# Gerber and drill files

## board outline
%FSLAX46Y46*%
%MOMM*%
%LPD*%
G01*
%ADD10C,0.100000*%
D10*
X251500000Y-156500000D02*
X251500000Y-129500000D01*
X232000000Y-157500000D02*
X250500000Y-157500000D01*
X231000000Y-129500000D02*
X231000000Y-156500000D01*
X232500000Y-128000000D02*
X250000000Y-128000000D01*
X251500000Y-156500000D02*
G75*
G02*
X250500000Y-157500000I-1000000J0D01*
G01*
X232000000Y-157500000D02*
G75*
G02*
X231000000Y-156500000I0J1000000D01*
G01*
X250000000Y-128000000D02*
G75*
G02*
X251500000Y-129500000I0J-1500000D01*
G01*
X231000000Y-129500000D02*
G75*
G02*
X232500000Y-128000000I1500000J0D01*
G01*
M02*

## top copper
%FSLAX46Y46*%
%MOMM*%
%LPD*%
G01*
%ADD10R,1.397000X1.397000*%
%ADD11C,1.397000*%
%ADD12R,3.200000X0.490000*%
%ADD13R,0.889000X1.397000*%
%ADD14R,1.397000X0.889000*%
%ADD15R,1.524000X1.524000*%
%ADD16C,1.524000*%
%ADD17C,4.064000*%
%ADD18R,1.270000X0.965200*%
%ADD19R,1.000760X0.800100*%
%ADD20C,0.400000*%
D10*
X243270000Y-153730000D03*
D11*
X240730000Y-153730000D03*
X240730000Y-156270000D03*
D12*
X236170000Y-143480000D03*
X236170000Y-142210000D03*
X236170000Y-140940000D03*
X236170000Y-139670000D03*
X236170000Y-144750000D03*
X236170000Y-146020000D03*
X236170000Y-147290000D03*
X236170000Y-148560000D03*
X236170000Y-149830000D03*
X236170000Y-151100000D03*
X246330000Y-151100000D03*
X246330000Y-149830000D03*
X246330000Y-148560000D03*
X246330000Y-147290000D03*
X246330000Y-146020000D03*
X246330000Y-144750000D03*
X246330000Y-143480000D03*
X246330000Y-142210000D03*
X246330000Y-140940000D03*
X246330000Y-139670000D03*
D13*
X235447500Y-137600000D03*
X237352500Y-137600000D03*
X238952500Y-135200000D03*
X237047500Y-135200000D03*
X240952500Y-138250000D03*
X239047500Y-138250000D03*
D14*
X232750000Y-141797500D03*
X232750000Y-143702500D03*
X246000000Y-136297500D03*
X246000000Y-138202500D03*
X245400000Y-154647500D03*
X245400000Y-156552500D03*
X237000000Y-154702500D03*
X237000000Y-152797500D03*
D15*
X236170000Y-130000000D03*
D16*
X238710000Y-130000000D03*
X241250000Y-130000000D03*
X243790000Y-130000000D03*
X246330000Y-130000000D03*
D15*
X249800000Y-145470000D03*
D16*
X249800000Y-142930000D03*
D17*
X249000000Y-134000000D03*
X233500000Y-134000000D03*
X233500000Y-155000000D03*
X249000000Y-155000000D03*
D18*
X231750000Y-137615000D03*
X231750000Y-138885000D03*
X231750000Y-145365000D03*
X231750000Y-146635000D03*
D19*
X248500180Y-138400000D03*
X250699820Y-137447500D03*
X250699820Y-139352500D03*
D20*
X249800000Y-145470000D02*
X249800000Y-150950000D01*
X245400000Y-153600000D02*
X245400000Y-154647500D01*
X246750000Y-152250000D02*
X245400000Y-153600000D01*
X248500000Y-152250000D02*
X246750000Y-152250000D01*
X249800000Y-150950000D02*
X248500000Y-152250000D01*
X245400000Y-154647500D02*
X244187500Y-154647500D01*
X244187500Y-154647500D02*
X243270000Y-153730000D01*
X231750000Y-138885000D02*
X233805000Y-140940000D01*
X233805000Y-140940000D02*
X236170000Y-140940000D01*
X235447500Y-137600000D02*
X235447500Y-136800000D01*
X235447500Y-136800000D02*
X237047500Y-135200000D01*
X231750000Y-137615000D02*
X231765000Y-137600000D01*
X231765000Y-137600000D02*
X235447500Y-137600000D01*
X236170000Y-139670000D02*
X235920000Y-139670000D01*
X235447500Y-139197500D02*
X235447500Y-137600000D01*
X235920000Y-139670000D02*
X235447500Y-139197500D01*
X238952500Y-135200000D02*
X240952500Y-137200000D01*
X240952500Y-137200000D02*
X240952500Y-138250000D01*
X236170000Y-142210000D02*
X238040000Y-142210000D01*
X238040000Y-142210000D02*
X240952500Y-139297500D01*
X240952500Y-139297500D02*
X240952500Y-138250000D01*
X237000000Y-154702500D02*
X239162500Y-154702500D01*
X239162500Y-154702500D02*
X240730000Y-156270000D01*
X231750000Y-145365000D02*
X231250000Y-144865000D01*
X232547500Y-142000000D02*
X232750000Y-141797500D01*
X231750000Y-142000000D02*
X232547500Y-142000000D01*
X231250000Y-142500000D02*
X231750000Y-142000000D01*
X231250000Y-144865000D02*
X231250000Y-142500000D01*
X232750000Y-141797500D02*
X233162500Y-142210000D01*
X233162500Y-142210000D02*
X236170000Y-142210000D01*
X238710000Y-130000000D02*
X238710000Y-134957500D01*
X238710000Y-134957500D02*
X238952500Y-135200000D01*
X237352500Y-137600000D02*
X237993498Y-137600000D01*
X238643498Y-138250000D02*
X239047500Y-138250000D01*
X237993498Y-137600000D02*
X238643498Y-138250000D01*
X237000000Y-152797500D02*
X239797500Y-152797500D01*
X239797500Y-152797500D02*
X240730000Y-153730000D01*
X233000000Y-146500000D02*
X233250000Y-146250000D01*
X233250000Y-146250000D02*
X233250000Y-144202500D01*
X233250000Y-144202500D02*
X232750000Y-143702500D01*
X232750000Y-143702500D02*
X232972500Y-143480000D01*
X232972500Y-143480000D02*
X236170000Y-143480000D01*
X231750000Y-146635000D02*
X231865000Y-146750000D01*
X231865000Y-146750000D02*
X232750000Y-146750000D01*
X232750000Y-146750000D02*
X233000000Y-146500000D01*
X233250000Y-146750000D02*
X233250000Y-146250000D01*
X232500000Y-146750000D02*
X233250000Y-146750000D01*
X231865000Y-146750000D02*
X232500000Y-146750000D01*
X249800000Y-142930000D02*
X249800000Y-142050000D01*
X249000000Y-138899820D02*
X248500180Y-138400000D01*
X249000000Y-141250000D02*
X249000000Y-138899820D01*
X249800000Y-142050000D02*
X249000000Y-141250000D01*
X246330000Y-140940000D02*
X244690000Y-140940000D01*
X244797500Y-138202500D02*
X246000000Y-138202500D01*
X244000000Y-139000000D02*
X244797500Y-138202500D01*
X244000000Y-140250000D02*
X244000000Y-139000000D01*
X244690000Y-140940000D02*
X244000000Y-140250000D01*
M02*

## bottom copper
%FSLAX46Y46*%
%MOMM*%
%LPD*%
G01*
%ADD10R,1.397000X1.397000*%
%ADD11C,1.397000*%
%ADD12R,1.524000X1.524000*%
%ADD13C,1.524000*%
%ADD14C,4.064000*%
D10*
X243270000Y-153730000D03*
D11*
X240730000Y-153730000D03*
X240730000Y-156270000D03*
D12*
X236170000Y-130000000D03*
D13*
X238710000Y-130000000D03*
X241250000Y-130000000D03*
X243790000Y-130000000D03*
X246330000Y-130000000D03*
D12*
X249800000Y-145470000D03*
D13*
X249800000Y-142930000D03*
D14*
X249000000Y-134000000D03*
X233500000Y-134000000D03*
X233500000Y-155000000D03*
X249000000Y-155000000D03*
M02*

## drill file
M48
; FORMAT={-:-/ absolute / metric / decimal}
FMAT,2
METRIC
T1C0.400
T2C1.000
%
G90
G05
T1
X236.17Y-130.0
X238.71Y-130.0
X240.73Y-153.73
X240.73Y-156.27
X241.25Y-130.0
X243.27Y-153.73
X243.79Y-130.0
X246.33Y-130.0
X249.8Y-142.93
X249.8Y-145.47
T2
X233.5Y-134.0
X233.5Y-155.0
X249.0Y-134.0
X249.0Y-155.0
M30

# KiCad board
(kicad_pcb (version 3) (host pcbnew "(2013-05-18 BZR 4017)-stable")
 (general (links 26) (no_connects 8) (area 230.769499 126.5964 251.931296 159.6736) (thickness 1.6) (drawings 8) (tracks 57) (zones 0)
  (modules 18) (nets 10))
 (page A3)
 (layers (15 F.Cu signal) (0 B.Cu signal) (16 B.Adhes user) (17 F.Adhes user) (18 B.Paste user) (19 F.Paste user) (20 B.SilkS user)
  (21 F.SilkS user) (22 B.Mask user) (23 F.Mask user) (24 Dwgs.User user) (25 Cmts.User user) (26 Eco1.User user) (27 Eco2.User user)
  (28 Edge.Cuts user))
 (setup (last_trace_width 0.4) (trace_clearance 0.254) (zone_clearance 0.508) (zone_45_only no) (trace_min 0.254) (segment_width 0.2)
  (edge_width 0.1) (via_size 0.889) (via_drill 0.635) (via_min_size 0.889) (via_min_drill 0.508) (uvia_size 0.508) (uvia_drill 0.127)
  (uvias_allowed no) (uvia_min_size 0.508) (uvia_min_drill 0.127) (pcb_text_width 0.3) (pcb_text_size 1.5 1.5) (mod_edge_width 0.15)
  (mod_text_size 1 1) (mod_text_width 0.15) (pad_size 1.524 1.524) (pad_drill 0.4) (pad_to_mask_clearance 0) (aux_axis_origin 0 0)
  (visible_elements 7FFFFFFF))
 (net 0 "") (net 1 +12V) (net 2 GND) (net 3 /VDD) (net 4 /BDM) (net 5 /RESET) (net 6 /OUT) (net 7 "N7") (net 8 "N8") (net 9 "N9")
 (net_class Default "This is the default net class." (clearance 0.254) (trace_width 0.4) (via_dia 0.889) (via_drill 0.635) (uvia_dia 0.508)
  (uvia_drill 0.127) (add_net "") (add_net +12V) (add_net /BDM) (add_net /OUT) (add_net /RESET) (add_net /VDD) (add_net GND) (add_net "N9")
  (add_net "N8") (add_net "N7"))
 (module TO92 (layer F.Cu) (at 242 155)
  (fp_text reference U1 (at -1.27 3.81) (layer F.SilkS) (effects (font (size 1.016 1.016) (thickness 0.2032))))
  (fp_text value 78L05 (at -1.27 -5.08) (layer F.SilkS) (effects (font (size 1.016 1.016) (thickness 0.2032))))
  (pad 1 thru_hole rect (at 1.27 -1.27) (size 1.397 1.397) (drill 0.4) (layers *.Cu *.Mask F.SilkS) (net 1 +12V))
  (pad 2 thru_hole circle (at -1.27 -1.27) (size 1.397 1.397) (drill 0.4) (layers *.Cu *.Mask F.SilkS) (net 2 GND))
  (pad 3 thru_hole circle (at -1.27 1.27) (size 1.397 1.397) (drill 0.4) (layers *.Cu *.Mask F.SilkS) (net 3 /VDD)))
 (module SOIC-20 (layer F.Cu) (at 241.25 144.75)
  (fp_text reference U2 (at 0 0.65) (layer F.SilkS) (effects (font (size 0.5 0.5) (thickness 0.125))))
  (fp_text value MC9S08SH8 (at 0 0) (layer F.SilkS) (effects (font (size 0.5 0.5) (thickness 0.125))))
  (pad 4 smd rect (at -5.08 -1.27) (size 3.2 0.49) (layers F.Cu F.Paste F.Mask) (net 2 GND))
  (pad 3 smd rect (at -5.08 -2.54) (size 3.2 0.49) (layers F.Cu F.Paste F.Mask) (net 3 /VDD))
  (pad 2 smd rect (at -5.08 -3.81) (size 3.2 0.49) (layers F.Cu F.Paste F.Mask) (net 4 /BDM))
  (pad 1 smd rect (at -5.08 -5.08) (size 3.2 0.49) (layers F.Cu F.Paste F.Mask) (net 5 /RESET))
  (pad 5 smd rect (at -5.08 0) (size 3.2 0.49) (layers F.Cu F.Paste F.Mask))
  (pad 6 smd rect (at -5.08 1.27) (size 3.2 0.49) (layers F.Cu F.Paste F.Mask))
  (pad 7 smd rect (at -5.08 2.54) (size 3.2 0.49) (layers F.Cu F.Paste F.Mask))
  (pad 8 smd rect (at -5.08 3.81) (size 3.2 0.49) (layers F.Cu F.Paste F.Mask))
  (pad 9 smd rect (at -5.08 5.08) (size 3.2 0.49) (layers F.Cu F.Paste F.Mask))
  (pad 10 smd rect (at -5.08 6.35) (size 3.2 0.49) (layers F.Cu F.Paste F.Mask))
  (pad 11 smd rect (at 5.08 6.35) (size 3.2 0.49) (layers F.Cu F.Paste F.Mask))
  (pad 12 smd rect (at 5.08 5.08) (size 3.2 0.49) (layers F.Cu F.Paste F.Mask) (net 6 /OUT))
  (pad 13 smd rect (at 5.08 3.81) (size 3.2 0.49) (layers F.Cu F.Paste F.Mask))
  (pad 14 smd rect (at 5.08 2.54) (size 3.2 0.49) (layers F.Cu F.Paste F.Mask))
  (pad 15 smd rect (at 5.08 1.27) (size 3.2 0.49) (layers F.Cu F.Paste F.Mask))
  (pad 16 smd rect (at 5.08 0) (size 3.2 0.49) (layers F.Cu F.Paste F.Mask))
  (pad 17 smd rect (at 5.08 -1.27) (size 3.2 0.49) (layers F.Cu F.Paste F.Mask))
  (pad 18 smd rect (at 5.08 -2.54) (size 3.2 0.49) (layers F.Cu F.Paste F.Mask))
  (pad 19 smd rect (at 5.08 -3.81) (size 3.2 0.49) (layers F.Cu F.Paste F.Mask) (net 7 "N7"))
  (pad 20 smd rect (at 5.08 -5.08) (size 3.2 0.49) (layers F.Cu F.Paste F.Mask)))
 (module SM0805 (layer F.Cu) (at 236.4 137.6)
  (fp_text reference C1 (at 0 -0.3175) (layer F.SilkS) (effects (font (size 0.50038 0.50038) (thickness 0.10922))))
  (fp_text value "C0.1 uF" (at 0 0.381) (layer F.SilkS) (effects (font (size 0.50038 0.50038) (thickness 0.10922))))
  (pad 1 smd rect (at -0.9525 0) (size 0.889 1.397) (layers F.Cu F.Paste F.Mask) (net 5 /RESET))
  (pad 2 smd rect (at 0.9525 0) (size 0.889 1.397) (layers F.Cu F.Paste F.Mask) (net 2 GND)))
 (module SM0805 (layer F.Cu) (at 238 135.2 180)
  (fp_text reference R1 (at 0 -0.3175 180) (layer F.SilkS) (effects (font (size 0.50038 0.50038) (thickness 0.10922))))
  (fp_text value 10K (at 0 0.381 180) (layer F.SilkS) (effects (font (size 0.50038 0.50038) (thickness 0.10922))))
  (pad 1 smd rect (at -0.9525 0 180) (size 0.889 1.397) (layers F.Cu F.Paste F.Mask) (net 3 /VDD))
  (pad 2 smd rect (at 0.9525 0 180) (size 0.889 1.397) (layers F.Cu F.Paste F.Mask) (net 5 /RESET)))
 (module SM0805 (layer F.Cu) (at 240 138.25 180)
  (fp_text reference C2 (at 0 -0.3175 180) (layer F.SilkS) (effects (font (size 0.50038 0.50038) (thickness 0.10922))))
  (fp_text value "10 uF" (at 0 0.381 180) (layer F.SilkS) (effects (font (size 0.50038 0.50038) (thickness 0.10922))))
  (pad 1 smd rect (at -0.9525 0 180) (size 0.889 1.397) (layers F.Cu F.Paste F.Mask) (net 3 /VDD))
  (pad 2 smd rect (at 0.9525 0 180) (size 0.889 1.397) (layers F.Cu F.Paste F.Mask) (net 2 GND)))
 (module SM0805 (layer F.Cu) (at 232.75 142.75 270)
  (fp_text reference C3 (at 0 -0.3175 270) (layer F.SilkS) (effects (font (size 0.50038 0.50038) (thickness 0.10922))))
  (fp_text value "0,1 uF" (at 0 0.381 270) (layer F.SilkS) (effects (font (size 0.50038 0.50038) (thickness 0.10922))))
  (pad 1 smd rect (at -0.9525 0 270) (size 0.889 1.397) (layers F.Cu F.Paste F.Mask) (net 3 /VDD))
  (pad 2 smd rect (at 0.9525 0 270) (size 0.889 1.397) (layers F.Cu F.Paste F.Mask) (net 2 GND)))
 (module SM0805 (layer F.Cu) (at 246 137.25 270)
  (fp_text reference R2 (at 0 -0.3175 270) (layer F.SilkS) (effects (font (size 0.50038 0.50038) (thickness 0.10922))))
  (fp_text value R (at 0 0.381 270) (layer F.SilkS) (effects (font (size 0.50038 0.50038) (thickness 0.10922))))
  (pad 1 smd rect (at -0.9525 0 270) (size 0.889 1.397) (layers F.Cu F.Paste F.Mask) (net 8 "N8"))
  (pad 2 smd rect (at 0.9525 0 270) (size 0.889 1.397) (layers F.Cu F.Paste F.Mask) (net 7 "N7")))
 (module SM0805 (layer F.Cu) (at 245.4 155.6 270)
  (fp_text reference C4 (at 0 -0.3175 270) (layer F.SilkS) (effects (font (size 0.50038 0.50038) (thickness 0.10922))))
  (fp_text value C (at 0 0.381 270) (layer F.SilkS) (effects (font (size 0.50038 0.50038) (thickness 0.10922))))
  (pad 1 smd rect (at -0.9525 0 270) (size 0.889 1.397) (layers F.Cu F.Paste F.Mask) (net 1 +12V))
  (pad 2 smd rect (at 0.9525 0 270) (size 0.889 1.397) (layers F.Cu F.Paste F.Mask) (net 2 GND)))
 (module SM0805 (layer F.Cu) (at 237 153.75 90)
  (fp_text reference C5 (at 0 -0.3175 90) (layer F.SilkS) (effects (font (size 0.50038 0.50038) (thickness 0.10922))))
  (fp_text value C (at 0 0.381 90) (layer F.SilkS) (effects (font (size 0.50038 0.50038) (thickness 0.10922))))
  (pad 1 smd rect (at -0.9525 0 90) (size 0.889 1.397) (layers F.Cu F.Paste F.Mask) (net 3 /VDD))
  (pad 2 smd rect (at 0.9525 0 90) (size 0.889 1.397) (layers F.Cu F.Paste F.Mask) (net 2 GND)))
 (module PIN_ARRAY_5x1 (layer F.Cu) (at 241.25 130)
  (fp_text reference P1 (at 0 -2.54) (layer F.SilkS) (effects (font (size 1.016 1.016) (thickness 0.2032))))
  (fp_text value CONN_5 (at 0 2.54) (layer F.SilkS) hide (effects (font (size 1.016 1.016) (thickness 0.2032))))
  (pad 1 thru_hole rect (at -5.08 0) (size 1.524 1.524) (drill 0.4) (layers *.Cu *.Mask F.SilkS))
  (pad 2 thru_hole circle (at -2.54 0) (size 1.524 1.524) (drill 0.4) (layers *.Cu *.Mask F.SilkS) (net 3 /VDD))
  (pad 3 thru_hole circle (at 0 0) (size 1.524 1.524) (drill 0.4) (layers *.Cu *.Mask F.SilkS))
  (pad 4 thru_hole circle (at 2.54 0) (size 1.524 1.524) (drill 0.4) (layers *.Cu *.Mask F.SilkS) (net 6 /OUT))
  (pad 5 thru_hole circle (at 5.08 0) (size 1.524 1.524) (drill 0.4) (layers *.Cu *.Mask F.SilkS) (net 2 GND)))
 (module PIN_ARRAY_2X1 (layer F.Cu) (at 249.8 144.2 90)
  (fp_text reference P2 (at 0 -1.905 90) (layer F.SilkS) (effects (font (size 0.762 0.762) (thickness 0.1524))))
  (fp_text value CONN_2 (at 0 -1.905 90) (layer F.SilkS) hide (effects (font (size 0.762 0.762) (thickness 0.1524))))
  (pad 1 thru_hole rect (at -1.27 0 90) (size 1.524 1.524) (drill 0.4) (layers *.Cu *.Mask F.SilkS) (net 1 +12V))
  (pad 2 thru_hole circle (at 1.27 0 90) (size 1.524 1.524) (drill 0.4) (layers *.Cu *.Mask F.SilkS) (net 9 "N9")))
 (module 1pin (layer F.Cu) (at 249 134)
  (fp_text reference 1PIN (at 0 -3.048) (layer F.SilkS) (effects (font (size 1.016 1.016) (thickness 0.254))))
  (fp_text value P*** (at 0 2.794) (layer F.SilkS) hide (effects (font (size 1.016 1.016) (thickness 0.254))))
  (pad 1 thru_hole circle (at 0 0) (size 4.064 4.064) (drill 1) (layers *.Cu *.Mask F.SilkS)))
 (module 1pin (layer F.Cu) (at 233.5 134)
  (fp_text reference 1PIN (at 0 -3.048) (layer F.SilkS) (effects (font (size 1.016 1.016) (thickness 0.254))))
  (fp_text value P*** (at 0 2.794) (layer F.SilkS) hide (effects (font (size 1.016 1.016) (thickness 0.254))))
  (pad 1 thru_hole circle (at 0 0) (size 4.064 4.064) (drill 1) (layers *.Cu *.Mask F.SilkS)))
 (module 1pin (layer F.Cu) (at 233.5 155)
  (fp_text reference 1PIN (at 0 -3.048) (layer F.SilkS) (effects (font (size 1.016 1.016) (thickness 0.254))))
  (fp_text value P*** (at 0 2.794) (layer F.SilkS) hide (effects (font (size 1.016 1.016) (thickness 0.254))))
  (pad 1 thru_hole circle (at 0 0) (size 4.064 4.064) (drill 1) (layers *.Cu *.Mask F.SilkS)))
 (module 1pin (layer F.Cu) (at 249 155)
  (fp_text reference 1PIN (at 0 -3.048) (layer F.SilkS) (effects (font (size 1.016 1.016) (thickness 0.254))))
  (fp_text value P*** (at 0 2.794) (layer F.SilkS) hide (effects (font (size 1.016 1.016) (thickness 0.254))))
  (pad 1 thru_hole circle (at 0 0) (size 4.064 4.064) (drill 1) (layers *.Cu *.Mask F.SilkS)))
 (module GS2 (layer F.Cu) (at 231.75 138.25)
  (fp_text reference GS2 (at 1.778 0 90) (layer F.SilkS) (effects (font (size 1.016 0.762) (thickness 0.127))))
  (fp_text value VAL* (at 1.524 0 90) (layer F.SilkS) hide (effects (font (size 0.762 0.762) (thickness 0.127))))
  (pad 1 smd rect (at 0 -0.635) (size 1.27 0.9652) (layers F.Cu F.Paste F.Mask) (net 5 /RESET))
  (pad 2 smd rect (at 0 0.635) (size 1.27 0.9652) (layers F.Cu F.Paste F.Mask) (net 4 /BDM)))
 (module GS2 (layer F.Cu) (at 231.75 146)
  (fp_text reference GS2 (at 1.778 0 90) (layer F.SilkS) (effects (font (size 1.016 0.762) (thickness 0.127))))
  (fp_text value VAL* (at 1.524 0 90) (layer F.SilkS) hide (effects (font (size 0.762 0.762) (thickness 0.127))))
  (pad 1 smd rect (at 0 -0.635) (size 1.27 0.9652) (layers F.Cu F.Paste F.Mask) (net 3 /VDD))
  (pad 2 smd rect (at 0 0.635) (size 1.27 0.9652) (layers F.Cu F.Paste F.Mask) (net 2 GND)))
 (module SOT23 (layer F.Cu) (at 249.6 138.4 90)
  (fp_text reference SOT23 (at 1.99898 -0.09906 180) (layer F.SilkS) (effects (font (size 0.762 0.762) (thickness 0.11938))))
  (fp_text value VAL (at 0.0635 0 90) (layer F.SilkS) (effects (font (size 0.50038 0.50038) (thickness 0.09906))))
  (pad 3 smd rect (at 0 -1.09982 90) (size 0.8001 1.00076) (layers F.Cu F.Paste F.Mask) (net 9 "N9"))
  (pad 2 smd rect (at 0.9525 1.09982 90) (size 0.8001 1.00076) (layers F.Cu F.Paste F.Mask) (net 2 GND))
  (pad 1 smd rect (at -0.9525 1.09982 90) (size 0.8001 1.00076) (layers F.Cu F.Paste F.Mask) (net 8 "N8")))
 (gr_line (start 251.5 156.5) (end 251.5 129.5) (angle 90) (layer Edge.Cuts) (width 0.1))
 (gr_line (start 232 157.5) (end 250.5 157.5) (angle 90) (layer Edge.Cuts) (width 0.1))
 (gr_line (start 231 129.5) (end 231 156.5) (angle 90) (layer Edge.Cuts) (width 0.1))
 (gr_line (start 232.5 128) (end 250 128) (angle 90) (layer Edge.Cuts) (width 0.1))
 (gr_arc (start 250.5 156.5) (end 251.5 156.5) (angle 90) (layer Edge.Cuts) (width 0.1))
 (gr_arc (start 232 156.5) (end 232 157.5) (angle 90) (layer Edge.Cuts) (width 0.1))
 (gr_arc (start 250 129.5) (end 250 128) (angle 90) (layer Edge.Cuts) (width 0.1))
 (gr_arc (start 232.5 129.5) (end 231 129.5) (angle 90) (layer Edge.Cuts) (width 0.1))
 (segment (start 249.8 145.47) (end 249.8 150.95) (width 0.4) (layer F.Cu) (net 1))
 (segment (start 245.4 153.6) (end 245.4 154.6475) (width 0.4) (layer F.Cu) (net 1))
 (segment (start 246.75 152.25) (end 245.4 153.6) (width 0.4) (layer F.Cu) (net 1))
 (segment (start 248.5 152.25) (end 246.75 152.25) (width 0.4) (layer F.Cu) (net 1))
 (segment (start 249.8 150.95) (end 248.5 152.25) (width 0.4) (layer F.Cu) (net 1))
 (segment (start 245.4 154.6475) (end 244.1875 154.6475) (width 0.4) (layer F.Cu) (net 1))
 (segment (start 244.1875 154.6475) (end 243.27 153.73) (width 0.4) (layer F.Cu) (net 1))
 (segment (start 231.75 138.885) (end 233.805 140.94) (width 0.4) (layer F.Cu) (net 4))
 (segment (start 233.805 140.94) (end 236.17 140.94) (width 0.4) (layer F.Cu) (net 4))
 (segment (start 235.4475 137.6) (end 235.4475 136.8) (width 0.4) (layer F.Cu) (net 5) (status 400000))
 (segment (start 235.4475 136.8) (end 237.0475 135.2) (width 0.4) (layer F.Cu) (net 5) (status 800000))
 (segment (start 231.75 137.615) (end 231.765 137.6) (width 0.4) (layer F.Cu) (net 5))
 (segment (start 231.765 137.6) (end 235.4475 137.6) (width 0.4) (layer F.Cu) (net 5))
 (segment (start 236.17 139.67) (end 235.92 139.67) (width 0.4) (layer F.Cu) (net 5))
 (segment (start 235.4475 139.1975) (end 235.4475 137.6) (width 0.4) (layer F.Cu) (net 5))
 (segment (start 235.92 139.67) (end 235.4475 139.1975) (width 0.4) (layer F.Cu) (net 5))
 (segment (start 238.9525 135.2) (end 240.9525 137.2) (width 0.4) (layer F.Cu) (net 3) (status 400000))
 (segment (start 240.9525 137.2) (end 240.9525 138.25) (width 0.4) (layer F.Cu) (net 3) (status 800000))
 (segment (start 236.17 142.21) (end 238.04 142.21) (width 0.4) (layer F.Cu) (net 3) (status 400000))
 (segment (start 238.04 142.21) (end 240.9525 139.2975) (width 0.4) (layer F.Cu) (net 3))
 (segment (start 240.9525 139.2975) (end 240.9525 138.25) (width 0.4) (layer F.Cu) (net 3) (status 800000))
 (segment (start 237 154.7025) (end 239.1625 154.7025) (width 0.4) (layer F.Cu) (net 3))
 (segment (start 239.1625 154.7025) (end 240.73 156.27) (width 0.4) (layer F.Cu) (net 3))
 (segment (start 231.75 145.365) (end 231.25 144.865) (width 0.4) (layer F.Cu) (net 3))
 (segment (start 232.5475 142) (end 232.75 141.7975) (width 0.4) (layer F.Cu) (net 3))
 (segment (start 231.75 142) (end 232.5475 142) (width 0.4) (layer F.Cu) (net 3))
 (segment (start 231.25 142.5) (end 231.75 142) (width 0.4) (layer F.Cu) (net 3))
 (segment (start 231.25 144.865) (end 231.25 142.5) (width 0.4) (layer F.Cu) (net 3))
 (segment (start 232.75 141.7975) (end 233.1625 142.21) (width 0.4) (layer F.Cu) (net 3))
 (segment (start 233.1625 142.21) (end 236.17 142.21) (width 0.4) (layer F.Cu) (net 3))
 (segment (start 238.71 130) (end 238.71 134.9575) (width 0.4) (layer F.Cu) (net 3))
 (segment (start 238.71 134.9575) (end 238.9525 135.2) (width 0.4) (layer F.Cu) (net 3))
 (segment (start 237.3525 137.6) (end 237.993498 137.6) (width 0.4) (layer F.Cu) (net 2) (status 400000))
 (segment (start 238.643498 138.25) (end 239.0475 138.25) (width 0.4) (layer F.Cu) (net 2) (status C00000))
 (segment (start 237.993498 137.6) (end 238.643498 138.25) (width 0.4) (layer F.Cu) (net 2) (status 800000))
 (segment (start 237 152.7975) (end 239.7975 152.7975) (width 0.4) (layer F.Cu) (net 2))
 (segment (start 239.7975 152.7975) (end 240.73 153.73) (width 0.4) (layer F.Cu) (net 2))
 (segment (start 233 146.5) (end 233.25 146.25) (width 0.4) (layer F.Cu) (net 2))
 (segment (start 233.25 146.25) (end 233.25 144.2025) (width 0.4) (layer F.Cu) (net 2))
 (segment (start 233.25 144.2025) (end 232.75 143.7025) (width 0.4) (layer F.Cu) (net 2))
 (segment (start 232.75 143.7025) (end 232.9725 143.48) (width 0.4) (layer F.Cu) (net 2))
 (segment (start 232.9725 143.48) (end 236.17 143.48) (width 0.4) (layer F.Cu) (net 2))
 (segment (start 231.75 146.635) (end 231.865 146.75) (width 0.4) (layer F.Cu) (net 2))
 (segment (start 231.865 146.75) (end 232.75 146.75) (width 0.4) (layer F.Cu) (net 2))
 (segment (start 232.75 146.75) (end 233 146.5) (width 0.4) (layer F.Cu) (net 2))
 (segment (start 233.25 146.75) (end 233.25 146.25) (width 0.4) (layer F.Cu) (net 2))
 (segment (start 232.5 146.75) (end 233.25 146.75) (width 0.4) (layer F.Cu) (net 2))
 (segment (start 231.865 146.75) (end 232.5 146.75) (width 0.4) (layer F.Cu) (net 2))
 (segment (start 249.8 142.93) (end 249.8 142.05) (width 0.4) (layer F.Cu) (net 9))
 (segment (start 249 138.89982) (end 248.50018 138.4) (width 0.4) (layer F.Cu) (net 9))
 (segment (start 249 141.25) (end 249 138.89982) (width 0.4) (layer F.Cu) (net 9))
 (segment (start 249.8 142.05) (end 249 141.25) (width 0.4) (layer F.Cu) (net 9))
 (segment (start 246.33 140.94) (end 244.69 140.94) (width 0.4) (layer F.Cu) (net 7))
 (segment (start 244.7975 138.2025) (end 246 138.2025) (width 0.4) (layer F.Cu) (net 7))
 (segment (start 244 139) (end 244.7975 138.2025) (width 0.4) (layer F.Cu) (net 7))
 (segment (start 244 140.25) (end 244 139) (width 0.4) (layer F.Cu) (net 7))
 (segment (start 244.69 140.94) (end 244 140.25) (width 0.4) (layer F.Cu) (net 7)))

